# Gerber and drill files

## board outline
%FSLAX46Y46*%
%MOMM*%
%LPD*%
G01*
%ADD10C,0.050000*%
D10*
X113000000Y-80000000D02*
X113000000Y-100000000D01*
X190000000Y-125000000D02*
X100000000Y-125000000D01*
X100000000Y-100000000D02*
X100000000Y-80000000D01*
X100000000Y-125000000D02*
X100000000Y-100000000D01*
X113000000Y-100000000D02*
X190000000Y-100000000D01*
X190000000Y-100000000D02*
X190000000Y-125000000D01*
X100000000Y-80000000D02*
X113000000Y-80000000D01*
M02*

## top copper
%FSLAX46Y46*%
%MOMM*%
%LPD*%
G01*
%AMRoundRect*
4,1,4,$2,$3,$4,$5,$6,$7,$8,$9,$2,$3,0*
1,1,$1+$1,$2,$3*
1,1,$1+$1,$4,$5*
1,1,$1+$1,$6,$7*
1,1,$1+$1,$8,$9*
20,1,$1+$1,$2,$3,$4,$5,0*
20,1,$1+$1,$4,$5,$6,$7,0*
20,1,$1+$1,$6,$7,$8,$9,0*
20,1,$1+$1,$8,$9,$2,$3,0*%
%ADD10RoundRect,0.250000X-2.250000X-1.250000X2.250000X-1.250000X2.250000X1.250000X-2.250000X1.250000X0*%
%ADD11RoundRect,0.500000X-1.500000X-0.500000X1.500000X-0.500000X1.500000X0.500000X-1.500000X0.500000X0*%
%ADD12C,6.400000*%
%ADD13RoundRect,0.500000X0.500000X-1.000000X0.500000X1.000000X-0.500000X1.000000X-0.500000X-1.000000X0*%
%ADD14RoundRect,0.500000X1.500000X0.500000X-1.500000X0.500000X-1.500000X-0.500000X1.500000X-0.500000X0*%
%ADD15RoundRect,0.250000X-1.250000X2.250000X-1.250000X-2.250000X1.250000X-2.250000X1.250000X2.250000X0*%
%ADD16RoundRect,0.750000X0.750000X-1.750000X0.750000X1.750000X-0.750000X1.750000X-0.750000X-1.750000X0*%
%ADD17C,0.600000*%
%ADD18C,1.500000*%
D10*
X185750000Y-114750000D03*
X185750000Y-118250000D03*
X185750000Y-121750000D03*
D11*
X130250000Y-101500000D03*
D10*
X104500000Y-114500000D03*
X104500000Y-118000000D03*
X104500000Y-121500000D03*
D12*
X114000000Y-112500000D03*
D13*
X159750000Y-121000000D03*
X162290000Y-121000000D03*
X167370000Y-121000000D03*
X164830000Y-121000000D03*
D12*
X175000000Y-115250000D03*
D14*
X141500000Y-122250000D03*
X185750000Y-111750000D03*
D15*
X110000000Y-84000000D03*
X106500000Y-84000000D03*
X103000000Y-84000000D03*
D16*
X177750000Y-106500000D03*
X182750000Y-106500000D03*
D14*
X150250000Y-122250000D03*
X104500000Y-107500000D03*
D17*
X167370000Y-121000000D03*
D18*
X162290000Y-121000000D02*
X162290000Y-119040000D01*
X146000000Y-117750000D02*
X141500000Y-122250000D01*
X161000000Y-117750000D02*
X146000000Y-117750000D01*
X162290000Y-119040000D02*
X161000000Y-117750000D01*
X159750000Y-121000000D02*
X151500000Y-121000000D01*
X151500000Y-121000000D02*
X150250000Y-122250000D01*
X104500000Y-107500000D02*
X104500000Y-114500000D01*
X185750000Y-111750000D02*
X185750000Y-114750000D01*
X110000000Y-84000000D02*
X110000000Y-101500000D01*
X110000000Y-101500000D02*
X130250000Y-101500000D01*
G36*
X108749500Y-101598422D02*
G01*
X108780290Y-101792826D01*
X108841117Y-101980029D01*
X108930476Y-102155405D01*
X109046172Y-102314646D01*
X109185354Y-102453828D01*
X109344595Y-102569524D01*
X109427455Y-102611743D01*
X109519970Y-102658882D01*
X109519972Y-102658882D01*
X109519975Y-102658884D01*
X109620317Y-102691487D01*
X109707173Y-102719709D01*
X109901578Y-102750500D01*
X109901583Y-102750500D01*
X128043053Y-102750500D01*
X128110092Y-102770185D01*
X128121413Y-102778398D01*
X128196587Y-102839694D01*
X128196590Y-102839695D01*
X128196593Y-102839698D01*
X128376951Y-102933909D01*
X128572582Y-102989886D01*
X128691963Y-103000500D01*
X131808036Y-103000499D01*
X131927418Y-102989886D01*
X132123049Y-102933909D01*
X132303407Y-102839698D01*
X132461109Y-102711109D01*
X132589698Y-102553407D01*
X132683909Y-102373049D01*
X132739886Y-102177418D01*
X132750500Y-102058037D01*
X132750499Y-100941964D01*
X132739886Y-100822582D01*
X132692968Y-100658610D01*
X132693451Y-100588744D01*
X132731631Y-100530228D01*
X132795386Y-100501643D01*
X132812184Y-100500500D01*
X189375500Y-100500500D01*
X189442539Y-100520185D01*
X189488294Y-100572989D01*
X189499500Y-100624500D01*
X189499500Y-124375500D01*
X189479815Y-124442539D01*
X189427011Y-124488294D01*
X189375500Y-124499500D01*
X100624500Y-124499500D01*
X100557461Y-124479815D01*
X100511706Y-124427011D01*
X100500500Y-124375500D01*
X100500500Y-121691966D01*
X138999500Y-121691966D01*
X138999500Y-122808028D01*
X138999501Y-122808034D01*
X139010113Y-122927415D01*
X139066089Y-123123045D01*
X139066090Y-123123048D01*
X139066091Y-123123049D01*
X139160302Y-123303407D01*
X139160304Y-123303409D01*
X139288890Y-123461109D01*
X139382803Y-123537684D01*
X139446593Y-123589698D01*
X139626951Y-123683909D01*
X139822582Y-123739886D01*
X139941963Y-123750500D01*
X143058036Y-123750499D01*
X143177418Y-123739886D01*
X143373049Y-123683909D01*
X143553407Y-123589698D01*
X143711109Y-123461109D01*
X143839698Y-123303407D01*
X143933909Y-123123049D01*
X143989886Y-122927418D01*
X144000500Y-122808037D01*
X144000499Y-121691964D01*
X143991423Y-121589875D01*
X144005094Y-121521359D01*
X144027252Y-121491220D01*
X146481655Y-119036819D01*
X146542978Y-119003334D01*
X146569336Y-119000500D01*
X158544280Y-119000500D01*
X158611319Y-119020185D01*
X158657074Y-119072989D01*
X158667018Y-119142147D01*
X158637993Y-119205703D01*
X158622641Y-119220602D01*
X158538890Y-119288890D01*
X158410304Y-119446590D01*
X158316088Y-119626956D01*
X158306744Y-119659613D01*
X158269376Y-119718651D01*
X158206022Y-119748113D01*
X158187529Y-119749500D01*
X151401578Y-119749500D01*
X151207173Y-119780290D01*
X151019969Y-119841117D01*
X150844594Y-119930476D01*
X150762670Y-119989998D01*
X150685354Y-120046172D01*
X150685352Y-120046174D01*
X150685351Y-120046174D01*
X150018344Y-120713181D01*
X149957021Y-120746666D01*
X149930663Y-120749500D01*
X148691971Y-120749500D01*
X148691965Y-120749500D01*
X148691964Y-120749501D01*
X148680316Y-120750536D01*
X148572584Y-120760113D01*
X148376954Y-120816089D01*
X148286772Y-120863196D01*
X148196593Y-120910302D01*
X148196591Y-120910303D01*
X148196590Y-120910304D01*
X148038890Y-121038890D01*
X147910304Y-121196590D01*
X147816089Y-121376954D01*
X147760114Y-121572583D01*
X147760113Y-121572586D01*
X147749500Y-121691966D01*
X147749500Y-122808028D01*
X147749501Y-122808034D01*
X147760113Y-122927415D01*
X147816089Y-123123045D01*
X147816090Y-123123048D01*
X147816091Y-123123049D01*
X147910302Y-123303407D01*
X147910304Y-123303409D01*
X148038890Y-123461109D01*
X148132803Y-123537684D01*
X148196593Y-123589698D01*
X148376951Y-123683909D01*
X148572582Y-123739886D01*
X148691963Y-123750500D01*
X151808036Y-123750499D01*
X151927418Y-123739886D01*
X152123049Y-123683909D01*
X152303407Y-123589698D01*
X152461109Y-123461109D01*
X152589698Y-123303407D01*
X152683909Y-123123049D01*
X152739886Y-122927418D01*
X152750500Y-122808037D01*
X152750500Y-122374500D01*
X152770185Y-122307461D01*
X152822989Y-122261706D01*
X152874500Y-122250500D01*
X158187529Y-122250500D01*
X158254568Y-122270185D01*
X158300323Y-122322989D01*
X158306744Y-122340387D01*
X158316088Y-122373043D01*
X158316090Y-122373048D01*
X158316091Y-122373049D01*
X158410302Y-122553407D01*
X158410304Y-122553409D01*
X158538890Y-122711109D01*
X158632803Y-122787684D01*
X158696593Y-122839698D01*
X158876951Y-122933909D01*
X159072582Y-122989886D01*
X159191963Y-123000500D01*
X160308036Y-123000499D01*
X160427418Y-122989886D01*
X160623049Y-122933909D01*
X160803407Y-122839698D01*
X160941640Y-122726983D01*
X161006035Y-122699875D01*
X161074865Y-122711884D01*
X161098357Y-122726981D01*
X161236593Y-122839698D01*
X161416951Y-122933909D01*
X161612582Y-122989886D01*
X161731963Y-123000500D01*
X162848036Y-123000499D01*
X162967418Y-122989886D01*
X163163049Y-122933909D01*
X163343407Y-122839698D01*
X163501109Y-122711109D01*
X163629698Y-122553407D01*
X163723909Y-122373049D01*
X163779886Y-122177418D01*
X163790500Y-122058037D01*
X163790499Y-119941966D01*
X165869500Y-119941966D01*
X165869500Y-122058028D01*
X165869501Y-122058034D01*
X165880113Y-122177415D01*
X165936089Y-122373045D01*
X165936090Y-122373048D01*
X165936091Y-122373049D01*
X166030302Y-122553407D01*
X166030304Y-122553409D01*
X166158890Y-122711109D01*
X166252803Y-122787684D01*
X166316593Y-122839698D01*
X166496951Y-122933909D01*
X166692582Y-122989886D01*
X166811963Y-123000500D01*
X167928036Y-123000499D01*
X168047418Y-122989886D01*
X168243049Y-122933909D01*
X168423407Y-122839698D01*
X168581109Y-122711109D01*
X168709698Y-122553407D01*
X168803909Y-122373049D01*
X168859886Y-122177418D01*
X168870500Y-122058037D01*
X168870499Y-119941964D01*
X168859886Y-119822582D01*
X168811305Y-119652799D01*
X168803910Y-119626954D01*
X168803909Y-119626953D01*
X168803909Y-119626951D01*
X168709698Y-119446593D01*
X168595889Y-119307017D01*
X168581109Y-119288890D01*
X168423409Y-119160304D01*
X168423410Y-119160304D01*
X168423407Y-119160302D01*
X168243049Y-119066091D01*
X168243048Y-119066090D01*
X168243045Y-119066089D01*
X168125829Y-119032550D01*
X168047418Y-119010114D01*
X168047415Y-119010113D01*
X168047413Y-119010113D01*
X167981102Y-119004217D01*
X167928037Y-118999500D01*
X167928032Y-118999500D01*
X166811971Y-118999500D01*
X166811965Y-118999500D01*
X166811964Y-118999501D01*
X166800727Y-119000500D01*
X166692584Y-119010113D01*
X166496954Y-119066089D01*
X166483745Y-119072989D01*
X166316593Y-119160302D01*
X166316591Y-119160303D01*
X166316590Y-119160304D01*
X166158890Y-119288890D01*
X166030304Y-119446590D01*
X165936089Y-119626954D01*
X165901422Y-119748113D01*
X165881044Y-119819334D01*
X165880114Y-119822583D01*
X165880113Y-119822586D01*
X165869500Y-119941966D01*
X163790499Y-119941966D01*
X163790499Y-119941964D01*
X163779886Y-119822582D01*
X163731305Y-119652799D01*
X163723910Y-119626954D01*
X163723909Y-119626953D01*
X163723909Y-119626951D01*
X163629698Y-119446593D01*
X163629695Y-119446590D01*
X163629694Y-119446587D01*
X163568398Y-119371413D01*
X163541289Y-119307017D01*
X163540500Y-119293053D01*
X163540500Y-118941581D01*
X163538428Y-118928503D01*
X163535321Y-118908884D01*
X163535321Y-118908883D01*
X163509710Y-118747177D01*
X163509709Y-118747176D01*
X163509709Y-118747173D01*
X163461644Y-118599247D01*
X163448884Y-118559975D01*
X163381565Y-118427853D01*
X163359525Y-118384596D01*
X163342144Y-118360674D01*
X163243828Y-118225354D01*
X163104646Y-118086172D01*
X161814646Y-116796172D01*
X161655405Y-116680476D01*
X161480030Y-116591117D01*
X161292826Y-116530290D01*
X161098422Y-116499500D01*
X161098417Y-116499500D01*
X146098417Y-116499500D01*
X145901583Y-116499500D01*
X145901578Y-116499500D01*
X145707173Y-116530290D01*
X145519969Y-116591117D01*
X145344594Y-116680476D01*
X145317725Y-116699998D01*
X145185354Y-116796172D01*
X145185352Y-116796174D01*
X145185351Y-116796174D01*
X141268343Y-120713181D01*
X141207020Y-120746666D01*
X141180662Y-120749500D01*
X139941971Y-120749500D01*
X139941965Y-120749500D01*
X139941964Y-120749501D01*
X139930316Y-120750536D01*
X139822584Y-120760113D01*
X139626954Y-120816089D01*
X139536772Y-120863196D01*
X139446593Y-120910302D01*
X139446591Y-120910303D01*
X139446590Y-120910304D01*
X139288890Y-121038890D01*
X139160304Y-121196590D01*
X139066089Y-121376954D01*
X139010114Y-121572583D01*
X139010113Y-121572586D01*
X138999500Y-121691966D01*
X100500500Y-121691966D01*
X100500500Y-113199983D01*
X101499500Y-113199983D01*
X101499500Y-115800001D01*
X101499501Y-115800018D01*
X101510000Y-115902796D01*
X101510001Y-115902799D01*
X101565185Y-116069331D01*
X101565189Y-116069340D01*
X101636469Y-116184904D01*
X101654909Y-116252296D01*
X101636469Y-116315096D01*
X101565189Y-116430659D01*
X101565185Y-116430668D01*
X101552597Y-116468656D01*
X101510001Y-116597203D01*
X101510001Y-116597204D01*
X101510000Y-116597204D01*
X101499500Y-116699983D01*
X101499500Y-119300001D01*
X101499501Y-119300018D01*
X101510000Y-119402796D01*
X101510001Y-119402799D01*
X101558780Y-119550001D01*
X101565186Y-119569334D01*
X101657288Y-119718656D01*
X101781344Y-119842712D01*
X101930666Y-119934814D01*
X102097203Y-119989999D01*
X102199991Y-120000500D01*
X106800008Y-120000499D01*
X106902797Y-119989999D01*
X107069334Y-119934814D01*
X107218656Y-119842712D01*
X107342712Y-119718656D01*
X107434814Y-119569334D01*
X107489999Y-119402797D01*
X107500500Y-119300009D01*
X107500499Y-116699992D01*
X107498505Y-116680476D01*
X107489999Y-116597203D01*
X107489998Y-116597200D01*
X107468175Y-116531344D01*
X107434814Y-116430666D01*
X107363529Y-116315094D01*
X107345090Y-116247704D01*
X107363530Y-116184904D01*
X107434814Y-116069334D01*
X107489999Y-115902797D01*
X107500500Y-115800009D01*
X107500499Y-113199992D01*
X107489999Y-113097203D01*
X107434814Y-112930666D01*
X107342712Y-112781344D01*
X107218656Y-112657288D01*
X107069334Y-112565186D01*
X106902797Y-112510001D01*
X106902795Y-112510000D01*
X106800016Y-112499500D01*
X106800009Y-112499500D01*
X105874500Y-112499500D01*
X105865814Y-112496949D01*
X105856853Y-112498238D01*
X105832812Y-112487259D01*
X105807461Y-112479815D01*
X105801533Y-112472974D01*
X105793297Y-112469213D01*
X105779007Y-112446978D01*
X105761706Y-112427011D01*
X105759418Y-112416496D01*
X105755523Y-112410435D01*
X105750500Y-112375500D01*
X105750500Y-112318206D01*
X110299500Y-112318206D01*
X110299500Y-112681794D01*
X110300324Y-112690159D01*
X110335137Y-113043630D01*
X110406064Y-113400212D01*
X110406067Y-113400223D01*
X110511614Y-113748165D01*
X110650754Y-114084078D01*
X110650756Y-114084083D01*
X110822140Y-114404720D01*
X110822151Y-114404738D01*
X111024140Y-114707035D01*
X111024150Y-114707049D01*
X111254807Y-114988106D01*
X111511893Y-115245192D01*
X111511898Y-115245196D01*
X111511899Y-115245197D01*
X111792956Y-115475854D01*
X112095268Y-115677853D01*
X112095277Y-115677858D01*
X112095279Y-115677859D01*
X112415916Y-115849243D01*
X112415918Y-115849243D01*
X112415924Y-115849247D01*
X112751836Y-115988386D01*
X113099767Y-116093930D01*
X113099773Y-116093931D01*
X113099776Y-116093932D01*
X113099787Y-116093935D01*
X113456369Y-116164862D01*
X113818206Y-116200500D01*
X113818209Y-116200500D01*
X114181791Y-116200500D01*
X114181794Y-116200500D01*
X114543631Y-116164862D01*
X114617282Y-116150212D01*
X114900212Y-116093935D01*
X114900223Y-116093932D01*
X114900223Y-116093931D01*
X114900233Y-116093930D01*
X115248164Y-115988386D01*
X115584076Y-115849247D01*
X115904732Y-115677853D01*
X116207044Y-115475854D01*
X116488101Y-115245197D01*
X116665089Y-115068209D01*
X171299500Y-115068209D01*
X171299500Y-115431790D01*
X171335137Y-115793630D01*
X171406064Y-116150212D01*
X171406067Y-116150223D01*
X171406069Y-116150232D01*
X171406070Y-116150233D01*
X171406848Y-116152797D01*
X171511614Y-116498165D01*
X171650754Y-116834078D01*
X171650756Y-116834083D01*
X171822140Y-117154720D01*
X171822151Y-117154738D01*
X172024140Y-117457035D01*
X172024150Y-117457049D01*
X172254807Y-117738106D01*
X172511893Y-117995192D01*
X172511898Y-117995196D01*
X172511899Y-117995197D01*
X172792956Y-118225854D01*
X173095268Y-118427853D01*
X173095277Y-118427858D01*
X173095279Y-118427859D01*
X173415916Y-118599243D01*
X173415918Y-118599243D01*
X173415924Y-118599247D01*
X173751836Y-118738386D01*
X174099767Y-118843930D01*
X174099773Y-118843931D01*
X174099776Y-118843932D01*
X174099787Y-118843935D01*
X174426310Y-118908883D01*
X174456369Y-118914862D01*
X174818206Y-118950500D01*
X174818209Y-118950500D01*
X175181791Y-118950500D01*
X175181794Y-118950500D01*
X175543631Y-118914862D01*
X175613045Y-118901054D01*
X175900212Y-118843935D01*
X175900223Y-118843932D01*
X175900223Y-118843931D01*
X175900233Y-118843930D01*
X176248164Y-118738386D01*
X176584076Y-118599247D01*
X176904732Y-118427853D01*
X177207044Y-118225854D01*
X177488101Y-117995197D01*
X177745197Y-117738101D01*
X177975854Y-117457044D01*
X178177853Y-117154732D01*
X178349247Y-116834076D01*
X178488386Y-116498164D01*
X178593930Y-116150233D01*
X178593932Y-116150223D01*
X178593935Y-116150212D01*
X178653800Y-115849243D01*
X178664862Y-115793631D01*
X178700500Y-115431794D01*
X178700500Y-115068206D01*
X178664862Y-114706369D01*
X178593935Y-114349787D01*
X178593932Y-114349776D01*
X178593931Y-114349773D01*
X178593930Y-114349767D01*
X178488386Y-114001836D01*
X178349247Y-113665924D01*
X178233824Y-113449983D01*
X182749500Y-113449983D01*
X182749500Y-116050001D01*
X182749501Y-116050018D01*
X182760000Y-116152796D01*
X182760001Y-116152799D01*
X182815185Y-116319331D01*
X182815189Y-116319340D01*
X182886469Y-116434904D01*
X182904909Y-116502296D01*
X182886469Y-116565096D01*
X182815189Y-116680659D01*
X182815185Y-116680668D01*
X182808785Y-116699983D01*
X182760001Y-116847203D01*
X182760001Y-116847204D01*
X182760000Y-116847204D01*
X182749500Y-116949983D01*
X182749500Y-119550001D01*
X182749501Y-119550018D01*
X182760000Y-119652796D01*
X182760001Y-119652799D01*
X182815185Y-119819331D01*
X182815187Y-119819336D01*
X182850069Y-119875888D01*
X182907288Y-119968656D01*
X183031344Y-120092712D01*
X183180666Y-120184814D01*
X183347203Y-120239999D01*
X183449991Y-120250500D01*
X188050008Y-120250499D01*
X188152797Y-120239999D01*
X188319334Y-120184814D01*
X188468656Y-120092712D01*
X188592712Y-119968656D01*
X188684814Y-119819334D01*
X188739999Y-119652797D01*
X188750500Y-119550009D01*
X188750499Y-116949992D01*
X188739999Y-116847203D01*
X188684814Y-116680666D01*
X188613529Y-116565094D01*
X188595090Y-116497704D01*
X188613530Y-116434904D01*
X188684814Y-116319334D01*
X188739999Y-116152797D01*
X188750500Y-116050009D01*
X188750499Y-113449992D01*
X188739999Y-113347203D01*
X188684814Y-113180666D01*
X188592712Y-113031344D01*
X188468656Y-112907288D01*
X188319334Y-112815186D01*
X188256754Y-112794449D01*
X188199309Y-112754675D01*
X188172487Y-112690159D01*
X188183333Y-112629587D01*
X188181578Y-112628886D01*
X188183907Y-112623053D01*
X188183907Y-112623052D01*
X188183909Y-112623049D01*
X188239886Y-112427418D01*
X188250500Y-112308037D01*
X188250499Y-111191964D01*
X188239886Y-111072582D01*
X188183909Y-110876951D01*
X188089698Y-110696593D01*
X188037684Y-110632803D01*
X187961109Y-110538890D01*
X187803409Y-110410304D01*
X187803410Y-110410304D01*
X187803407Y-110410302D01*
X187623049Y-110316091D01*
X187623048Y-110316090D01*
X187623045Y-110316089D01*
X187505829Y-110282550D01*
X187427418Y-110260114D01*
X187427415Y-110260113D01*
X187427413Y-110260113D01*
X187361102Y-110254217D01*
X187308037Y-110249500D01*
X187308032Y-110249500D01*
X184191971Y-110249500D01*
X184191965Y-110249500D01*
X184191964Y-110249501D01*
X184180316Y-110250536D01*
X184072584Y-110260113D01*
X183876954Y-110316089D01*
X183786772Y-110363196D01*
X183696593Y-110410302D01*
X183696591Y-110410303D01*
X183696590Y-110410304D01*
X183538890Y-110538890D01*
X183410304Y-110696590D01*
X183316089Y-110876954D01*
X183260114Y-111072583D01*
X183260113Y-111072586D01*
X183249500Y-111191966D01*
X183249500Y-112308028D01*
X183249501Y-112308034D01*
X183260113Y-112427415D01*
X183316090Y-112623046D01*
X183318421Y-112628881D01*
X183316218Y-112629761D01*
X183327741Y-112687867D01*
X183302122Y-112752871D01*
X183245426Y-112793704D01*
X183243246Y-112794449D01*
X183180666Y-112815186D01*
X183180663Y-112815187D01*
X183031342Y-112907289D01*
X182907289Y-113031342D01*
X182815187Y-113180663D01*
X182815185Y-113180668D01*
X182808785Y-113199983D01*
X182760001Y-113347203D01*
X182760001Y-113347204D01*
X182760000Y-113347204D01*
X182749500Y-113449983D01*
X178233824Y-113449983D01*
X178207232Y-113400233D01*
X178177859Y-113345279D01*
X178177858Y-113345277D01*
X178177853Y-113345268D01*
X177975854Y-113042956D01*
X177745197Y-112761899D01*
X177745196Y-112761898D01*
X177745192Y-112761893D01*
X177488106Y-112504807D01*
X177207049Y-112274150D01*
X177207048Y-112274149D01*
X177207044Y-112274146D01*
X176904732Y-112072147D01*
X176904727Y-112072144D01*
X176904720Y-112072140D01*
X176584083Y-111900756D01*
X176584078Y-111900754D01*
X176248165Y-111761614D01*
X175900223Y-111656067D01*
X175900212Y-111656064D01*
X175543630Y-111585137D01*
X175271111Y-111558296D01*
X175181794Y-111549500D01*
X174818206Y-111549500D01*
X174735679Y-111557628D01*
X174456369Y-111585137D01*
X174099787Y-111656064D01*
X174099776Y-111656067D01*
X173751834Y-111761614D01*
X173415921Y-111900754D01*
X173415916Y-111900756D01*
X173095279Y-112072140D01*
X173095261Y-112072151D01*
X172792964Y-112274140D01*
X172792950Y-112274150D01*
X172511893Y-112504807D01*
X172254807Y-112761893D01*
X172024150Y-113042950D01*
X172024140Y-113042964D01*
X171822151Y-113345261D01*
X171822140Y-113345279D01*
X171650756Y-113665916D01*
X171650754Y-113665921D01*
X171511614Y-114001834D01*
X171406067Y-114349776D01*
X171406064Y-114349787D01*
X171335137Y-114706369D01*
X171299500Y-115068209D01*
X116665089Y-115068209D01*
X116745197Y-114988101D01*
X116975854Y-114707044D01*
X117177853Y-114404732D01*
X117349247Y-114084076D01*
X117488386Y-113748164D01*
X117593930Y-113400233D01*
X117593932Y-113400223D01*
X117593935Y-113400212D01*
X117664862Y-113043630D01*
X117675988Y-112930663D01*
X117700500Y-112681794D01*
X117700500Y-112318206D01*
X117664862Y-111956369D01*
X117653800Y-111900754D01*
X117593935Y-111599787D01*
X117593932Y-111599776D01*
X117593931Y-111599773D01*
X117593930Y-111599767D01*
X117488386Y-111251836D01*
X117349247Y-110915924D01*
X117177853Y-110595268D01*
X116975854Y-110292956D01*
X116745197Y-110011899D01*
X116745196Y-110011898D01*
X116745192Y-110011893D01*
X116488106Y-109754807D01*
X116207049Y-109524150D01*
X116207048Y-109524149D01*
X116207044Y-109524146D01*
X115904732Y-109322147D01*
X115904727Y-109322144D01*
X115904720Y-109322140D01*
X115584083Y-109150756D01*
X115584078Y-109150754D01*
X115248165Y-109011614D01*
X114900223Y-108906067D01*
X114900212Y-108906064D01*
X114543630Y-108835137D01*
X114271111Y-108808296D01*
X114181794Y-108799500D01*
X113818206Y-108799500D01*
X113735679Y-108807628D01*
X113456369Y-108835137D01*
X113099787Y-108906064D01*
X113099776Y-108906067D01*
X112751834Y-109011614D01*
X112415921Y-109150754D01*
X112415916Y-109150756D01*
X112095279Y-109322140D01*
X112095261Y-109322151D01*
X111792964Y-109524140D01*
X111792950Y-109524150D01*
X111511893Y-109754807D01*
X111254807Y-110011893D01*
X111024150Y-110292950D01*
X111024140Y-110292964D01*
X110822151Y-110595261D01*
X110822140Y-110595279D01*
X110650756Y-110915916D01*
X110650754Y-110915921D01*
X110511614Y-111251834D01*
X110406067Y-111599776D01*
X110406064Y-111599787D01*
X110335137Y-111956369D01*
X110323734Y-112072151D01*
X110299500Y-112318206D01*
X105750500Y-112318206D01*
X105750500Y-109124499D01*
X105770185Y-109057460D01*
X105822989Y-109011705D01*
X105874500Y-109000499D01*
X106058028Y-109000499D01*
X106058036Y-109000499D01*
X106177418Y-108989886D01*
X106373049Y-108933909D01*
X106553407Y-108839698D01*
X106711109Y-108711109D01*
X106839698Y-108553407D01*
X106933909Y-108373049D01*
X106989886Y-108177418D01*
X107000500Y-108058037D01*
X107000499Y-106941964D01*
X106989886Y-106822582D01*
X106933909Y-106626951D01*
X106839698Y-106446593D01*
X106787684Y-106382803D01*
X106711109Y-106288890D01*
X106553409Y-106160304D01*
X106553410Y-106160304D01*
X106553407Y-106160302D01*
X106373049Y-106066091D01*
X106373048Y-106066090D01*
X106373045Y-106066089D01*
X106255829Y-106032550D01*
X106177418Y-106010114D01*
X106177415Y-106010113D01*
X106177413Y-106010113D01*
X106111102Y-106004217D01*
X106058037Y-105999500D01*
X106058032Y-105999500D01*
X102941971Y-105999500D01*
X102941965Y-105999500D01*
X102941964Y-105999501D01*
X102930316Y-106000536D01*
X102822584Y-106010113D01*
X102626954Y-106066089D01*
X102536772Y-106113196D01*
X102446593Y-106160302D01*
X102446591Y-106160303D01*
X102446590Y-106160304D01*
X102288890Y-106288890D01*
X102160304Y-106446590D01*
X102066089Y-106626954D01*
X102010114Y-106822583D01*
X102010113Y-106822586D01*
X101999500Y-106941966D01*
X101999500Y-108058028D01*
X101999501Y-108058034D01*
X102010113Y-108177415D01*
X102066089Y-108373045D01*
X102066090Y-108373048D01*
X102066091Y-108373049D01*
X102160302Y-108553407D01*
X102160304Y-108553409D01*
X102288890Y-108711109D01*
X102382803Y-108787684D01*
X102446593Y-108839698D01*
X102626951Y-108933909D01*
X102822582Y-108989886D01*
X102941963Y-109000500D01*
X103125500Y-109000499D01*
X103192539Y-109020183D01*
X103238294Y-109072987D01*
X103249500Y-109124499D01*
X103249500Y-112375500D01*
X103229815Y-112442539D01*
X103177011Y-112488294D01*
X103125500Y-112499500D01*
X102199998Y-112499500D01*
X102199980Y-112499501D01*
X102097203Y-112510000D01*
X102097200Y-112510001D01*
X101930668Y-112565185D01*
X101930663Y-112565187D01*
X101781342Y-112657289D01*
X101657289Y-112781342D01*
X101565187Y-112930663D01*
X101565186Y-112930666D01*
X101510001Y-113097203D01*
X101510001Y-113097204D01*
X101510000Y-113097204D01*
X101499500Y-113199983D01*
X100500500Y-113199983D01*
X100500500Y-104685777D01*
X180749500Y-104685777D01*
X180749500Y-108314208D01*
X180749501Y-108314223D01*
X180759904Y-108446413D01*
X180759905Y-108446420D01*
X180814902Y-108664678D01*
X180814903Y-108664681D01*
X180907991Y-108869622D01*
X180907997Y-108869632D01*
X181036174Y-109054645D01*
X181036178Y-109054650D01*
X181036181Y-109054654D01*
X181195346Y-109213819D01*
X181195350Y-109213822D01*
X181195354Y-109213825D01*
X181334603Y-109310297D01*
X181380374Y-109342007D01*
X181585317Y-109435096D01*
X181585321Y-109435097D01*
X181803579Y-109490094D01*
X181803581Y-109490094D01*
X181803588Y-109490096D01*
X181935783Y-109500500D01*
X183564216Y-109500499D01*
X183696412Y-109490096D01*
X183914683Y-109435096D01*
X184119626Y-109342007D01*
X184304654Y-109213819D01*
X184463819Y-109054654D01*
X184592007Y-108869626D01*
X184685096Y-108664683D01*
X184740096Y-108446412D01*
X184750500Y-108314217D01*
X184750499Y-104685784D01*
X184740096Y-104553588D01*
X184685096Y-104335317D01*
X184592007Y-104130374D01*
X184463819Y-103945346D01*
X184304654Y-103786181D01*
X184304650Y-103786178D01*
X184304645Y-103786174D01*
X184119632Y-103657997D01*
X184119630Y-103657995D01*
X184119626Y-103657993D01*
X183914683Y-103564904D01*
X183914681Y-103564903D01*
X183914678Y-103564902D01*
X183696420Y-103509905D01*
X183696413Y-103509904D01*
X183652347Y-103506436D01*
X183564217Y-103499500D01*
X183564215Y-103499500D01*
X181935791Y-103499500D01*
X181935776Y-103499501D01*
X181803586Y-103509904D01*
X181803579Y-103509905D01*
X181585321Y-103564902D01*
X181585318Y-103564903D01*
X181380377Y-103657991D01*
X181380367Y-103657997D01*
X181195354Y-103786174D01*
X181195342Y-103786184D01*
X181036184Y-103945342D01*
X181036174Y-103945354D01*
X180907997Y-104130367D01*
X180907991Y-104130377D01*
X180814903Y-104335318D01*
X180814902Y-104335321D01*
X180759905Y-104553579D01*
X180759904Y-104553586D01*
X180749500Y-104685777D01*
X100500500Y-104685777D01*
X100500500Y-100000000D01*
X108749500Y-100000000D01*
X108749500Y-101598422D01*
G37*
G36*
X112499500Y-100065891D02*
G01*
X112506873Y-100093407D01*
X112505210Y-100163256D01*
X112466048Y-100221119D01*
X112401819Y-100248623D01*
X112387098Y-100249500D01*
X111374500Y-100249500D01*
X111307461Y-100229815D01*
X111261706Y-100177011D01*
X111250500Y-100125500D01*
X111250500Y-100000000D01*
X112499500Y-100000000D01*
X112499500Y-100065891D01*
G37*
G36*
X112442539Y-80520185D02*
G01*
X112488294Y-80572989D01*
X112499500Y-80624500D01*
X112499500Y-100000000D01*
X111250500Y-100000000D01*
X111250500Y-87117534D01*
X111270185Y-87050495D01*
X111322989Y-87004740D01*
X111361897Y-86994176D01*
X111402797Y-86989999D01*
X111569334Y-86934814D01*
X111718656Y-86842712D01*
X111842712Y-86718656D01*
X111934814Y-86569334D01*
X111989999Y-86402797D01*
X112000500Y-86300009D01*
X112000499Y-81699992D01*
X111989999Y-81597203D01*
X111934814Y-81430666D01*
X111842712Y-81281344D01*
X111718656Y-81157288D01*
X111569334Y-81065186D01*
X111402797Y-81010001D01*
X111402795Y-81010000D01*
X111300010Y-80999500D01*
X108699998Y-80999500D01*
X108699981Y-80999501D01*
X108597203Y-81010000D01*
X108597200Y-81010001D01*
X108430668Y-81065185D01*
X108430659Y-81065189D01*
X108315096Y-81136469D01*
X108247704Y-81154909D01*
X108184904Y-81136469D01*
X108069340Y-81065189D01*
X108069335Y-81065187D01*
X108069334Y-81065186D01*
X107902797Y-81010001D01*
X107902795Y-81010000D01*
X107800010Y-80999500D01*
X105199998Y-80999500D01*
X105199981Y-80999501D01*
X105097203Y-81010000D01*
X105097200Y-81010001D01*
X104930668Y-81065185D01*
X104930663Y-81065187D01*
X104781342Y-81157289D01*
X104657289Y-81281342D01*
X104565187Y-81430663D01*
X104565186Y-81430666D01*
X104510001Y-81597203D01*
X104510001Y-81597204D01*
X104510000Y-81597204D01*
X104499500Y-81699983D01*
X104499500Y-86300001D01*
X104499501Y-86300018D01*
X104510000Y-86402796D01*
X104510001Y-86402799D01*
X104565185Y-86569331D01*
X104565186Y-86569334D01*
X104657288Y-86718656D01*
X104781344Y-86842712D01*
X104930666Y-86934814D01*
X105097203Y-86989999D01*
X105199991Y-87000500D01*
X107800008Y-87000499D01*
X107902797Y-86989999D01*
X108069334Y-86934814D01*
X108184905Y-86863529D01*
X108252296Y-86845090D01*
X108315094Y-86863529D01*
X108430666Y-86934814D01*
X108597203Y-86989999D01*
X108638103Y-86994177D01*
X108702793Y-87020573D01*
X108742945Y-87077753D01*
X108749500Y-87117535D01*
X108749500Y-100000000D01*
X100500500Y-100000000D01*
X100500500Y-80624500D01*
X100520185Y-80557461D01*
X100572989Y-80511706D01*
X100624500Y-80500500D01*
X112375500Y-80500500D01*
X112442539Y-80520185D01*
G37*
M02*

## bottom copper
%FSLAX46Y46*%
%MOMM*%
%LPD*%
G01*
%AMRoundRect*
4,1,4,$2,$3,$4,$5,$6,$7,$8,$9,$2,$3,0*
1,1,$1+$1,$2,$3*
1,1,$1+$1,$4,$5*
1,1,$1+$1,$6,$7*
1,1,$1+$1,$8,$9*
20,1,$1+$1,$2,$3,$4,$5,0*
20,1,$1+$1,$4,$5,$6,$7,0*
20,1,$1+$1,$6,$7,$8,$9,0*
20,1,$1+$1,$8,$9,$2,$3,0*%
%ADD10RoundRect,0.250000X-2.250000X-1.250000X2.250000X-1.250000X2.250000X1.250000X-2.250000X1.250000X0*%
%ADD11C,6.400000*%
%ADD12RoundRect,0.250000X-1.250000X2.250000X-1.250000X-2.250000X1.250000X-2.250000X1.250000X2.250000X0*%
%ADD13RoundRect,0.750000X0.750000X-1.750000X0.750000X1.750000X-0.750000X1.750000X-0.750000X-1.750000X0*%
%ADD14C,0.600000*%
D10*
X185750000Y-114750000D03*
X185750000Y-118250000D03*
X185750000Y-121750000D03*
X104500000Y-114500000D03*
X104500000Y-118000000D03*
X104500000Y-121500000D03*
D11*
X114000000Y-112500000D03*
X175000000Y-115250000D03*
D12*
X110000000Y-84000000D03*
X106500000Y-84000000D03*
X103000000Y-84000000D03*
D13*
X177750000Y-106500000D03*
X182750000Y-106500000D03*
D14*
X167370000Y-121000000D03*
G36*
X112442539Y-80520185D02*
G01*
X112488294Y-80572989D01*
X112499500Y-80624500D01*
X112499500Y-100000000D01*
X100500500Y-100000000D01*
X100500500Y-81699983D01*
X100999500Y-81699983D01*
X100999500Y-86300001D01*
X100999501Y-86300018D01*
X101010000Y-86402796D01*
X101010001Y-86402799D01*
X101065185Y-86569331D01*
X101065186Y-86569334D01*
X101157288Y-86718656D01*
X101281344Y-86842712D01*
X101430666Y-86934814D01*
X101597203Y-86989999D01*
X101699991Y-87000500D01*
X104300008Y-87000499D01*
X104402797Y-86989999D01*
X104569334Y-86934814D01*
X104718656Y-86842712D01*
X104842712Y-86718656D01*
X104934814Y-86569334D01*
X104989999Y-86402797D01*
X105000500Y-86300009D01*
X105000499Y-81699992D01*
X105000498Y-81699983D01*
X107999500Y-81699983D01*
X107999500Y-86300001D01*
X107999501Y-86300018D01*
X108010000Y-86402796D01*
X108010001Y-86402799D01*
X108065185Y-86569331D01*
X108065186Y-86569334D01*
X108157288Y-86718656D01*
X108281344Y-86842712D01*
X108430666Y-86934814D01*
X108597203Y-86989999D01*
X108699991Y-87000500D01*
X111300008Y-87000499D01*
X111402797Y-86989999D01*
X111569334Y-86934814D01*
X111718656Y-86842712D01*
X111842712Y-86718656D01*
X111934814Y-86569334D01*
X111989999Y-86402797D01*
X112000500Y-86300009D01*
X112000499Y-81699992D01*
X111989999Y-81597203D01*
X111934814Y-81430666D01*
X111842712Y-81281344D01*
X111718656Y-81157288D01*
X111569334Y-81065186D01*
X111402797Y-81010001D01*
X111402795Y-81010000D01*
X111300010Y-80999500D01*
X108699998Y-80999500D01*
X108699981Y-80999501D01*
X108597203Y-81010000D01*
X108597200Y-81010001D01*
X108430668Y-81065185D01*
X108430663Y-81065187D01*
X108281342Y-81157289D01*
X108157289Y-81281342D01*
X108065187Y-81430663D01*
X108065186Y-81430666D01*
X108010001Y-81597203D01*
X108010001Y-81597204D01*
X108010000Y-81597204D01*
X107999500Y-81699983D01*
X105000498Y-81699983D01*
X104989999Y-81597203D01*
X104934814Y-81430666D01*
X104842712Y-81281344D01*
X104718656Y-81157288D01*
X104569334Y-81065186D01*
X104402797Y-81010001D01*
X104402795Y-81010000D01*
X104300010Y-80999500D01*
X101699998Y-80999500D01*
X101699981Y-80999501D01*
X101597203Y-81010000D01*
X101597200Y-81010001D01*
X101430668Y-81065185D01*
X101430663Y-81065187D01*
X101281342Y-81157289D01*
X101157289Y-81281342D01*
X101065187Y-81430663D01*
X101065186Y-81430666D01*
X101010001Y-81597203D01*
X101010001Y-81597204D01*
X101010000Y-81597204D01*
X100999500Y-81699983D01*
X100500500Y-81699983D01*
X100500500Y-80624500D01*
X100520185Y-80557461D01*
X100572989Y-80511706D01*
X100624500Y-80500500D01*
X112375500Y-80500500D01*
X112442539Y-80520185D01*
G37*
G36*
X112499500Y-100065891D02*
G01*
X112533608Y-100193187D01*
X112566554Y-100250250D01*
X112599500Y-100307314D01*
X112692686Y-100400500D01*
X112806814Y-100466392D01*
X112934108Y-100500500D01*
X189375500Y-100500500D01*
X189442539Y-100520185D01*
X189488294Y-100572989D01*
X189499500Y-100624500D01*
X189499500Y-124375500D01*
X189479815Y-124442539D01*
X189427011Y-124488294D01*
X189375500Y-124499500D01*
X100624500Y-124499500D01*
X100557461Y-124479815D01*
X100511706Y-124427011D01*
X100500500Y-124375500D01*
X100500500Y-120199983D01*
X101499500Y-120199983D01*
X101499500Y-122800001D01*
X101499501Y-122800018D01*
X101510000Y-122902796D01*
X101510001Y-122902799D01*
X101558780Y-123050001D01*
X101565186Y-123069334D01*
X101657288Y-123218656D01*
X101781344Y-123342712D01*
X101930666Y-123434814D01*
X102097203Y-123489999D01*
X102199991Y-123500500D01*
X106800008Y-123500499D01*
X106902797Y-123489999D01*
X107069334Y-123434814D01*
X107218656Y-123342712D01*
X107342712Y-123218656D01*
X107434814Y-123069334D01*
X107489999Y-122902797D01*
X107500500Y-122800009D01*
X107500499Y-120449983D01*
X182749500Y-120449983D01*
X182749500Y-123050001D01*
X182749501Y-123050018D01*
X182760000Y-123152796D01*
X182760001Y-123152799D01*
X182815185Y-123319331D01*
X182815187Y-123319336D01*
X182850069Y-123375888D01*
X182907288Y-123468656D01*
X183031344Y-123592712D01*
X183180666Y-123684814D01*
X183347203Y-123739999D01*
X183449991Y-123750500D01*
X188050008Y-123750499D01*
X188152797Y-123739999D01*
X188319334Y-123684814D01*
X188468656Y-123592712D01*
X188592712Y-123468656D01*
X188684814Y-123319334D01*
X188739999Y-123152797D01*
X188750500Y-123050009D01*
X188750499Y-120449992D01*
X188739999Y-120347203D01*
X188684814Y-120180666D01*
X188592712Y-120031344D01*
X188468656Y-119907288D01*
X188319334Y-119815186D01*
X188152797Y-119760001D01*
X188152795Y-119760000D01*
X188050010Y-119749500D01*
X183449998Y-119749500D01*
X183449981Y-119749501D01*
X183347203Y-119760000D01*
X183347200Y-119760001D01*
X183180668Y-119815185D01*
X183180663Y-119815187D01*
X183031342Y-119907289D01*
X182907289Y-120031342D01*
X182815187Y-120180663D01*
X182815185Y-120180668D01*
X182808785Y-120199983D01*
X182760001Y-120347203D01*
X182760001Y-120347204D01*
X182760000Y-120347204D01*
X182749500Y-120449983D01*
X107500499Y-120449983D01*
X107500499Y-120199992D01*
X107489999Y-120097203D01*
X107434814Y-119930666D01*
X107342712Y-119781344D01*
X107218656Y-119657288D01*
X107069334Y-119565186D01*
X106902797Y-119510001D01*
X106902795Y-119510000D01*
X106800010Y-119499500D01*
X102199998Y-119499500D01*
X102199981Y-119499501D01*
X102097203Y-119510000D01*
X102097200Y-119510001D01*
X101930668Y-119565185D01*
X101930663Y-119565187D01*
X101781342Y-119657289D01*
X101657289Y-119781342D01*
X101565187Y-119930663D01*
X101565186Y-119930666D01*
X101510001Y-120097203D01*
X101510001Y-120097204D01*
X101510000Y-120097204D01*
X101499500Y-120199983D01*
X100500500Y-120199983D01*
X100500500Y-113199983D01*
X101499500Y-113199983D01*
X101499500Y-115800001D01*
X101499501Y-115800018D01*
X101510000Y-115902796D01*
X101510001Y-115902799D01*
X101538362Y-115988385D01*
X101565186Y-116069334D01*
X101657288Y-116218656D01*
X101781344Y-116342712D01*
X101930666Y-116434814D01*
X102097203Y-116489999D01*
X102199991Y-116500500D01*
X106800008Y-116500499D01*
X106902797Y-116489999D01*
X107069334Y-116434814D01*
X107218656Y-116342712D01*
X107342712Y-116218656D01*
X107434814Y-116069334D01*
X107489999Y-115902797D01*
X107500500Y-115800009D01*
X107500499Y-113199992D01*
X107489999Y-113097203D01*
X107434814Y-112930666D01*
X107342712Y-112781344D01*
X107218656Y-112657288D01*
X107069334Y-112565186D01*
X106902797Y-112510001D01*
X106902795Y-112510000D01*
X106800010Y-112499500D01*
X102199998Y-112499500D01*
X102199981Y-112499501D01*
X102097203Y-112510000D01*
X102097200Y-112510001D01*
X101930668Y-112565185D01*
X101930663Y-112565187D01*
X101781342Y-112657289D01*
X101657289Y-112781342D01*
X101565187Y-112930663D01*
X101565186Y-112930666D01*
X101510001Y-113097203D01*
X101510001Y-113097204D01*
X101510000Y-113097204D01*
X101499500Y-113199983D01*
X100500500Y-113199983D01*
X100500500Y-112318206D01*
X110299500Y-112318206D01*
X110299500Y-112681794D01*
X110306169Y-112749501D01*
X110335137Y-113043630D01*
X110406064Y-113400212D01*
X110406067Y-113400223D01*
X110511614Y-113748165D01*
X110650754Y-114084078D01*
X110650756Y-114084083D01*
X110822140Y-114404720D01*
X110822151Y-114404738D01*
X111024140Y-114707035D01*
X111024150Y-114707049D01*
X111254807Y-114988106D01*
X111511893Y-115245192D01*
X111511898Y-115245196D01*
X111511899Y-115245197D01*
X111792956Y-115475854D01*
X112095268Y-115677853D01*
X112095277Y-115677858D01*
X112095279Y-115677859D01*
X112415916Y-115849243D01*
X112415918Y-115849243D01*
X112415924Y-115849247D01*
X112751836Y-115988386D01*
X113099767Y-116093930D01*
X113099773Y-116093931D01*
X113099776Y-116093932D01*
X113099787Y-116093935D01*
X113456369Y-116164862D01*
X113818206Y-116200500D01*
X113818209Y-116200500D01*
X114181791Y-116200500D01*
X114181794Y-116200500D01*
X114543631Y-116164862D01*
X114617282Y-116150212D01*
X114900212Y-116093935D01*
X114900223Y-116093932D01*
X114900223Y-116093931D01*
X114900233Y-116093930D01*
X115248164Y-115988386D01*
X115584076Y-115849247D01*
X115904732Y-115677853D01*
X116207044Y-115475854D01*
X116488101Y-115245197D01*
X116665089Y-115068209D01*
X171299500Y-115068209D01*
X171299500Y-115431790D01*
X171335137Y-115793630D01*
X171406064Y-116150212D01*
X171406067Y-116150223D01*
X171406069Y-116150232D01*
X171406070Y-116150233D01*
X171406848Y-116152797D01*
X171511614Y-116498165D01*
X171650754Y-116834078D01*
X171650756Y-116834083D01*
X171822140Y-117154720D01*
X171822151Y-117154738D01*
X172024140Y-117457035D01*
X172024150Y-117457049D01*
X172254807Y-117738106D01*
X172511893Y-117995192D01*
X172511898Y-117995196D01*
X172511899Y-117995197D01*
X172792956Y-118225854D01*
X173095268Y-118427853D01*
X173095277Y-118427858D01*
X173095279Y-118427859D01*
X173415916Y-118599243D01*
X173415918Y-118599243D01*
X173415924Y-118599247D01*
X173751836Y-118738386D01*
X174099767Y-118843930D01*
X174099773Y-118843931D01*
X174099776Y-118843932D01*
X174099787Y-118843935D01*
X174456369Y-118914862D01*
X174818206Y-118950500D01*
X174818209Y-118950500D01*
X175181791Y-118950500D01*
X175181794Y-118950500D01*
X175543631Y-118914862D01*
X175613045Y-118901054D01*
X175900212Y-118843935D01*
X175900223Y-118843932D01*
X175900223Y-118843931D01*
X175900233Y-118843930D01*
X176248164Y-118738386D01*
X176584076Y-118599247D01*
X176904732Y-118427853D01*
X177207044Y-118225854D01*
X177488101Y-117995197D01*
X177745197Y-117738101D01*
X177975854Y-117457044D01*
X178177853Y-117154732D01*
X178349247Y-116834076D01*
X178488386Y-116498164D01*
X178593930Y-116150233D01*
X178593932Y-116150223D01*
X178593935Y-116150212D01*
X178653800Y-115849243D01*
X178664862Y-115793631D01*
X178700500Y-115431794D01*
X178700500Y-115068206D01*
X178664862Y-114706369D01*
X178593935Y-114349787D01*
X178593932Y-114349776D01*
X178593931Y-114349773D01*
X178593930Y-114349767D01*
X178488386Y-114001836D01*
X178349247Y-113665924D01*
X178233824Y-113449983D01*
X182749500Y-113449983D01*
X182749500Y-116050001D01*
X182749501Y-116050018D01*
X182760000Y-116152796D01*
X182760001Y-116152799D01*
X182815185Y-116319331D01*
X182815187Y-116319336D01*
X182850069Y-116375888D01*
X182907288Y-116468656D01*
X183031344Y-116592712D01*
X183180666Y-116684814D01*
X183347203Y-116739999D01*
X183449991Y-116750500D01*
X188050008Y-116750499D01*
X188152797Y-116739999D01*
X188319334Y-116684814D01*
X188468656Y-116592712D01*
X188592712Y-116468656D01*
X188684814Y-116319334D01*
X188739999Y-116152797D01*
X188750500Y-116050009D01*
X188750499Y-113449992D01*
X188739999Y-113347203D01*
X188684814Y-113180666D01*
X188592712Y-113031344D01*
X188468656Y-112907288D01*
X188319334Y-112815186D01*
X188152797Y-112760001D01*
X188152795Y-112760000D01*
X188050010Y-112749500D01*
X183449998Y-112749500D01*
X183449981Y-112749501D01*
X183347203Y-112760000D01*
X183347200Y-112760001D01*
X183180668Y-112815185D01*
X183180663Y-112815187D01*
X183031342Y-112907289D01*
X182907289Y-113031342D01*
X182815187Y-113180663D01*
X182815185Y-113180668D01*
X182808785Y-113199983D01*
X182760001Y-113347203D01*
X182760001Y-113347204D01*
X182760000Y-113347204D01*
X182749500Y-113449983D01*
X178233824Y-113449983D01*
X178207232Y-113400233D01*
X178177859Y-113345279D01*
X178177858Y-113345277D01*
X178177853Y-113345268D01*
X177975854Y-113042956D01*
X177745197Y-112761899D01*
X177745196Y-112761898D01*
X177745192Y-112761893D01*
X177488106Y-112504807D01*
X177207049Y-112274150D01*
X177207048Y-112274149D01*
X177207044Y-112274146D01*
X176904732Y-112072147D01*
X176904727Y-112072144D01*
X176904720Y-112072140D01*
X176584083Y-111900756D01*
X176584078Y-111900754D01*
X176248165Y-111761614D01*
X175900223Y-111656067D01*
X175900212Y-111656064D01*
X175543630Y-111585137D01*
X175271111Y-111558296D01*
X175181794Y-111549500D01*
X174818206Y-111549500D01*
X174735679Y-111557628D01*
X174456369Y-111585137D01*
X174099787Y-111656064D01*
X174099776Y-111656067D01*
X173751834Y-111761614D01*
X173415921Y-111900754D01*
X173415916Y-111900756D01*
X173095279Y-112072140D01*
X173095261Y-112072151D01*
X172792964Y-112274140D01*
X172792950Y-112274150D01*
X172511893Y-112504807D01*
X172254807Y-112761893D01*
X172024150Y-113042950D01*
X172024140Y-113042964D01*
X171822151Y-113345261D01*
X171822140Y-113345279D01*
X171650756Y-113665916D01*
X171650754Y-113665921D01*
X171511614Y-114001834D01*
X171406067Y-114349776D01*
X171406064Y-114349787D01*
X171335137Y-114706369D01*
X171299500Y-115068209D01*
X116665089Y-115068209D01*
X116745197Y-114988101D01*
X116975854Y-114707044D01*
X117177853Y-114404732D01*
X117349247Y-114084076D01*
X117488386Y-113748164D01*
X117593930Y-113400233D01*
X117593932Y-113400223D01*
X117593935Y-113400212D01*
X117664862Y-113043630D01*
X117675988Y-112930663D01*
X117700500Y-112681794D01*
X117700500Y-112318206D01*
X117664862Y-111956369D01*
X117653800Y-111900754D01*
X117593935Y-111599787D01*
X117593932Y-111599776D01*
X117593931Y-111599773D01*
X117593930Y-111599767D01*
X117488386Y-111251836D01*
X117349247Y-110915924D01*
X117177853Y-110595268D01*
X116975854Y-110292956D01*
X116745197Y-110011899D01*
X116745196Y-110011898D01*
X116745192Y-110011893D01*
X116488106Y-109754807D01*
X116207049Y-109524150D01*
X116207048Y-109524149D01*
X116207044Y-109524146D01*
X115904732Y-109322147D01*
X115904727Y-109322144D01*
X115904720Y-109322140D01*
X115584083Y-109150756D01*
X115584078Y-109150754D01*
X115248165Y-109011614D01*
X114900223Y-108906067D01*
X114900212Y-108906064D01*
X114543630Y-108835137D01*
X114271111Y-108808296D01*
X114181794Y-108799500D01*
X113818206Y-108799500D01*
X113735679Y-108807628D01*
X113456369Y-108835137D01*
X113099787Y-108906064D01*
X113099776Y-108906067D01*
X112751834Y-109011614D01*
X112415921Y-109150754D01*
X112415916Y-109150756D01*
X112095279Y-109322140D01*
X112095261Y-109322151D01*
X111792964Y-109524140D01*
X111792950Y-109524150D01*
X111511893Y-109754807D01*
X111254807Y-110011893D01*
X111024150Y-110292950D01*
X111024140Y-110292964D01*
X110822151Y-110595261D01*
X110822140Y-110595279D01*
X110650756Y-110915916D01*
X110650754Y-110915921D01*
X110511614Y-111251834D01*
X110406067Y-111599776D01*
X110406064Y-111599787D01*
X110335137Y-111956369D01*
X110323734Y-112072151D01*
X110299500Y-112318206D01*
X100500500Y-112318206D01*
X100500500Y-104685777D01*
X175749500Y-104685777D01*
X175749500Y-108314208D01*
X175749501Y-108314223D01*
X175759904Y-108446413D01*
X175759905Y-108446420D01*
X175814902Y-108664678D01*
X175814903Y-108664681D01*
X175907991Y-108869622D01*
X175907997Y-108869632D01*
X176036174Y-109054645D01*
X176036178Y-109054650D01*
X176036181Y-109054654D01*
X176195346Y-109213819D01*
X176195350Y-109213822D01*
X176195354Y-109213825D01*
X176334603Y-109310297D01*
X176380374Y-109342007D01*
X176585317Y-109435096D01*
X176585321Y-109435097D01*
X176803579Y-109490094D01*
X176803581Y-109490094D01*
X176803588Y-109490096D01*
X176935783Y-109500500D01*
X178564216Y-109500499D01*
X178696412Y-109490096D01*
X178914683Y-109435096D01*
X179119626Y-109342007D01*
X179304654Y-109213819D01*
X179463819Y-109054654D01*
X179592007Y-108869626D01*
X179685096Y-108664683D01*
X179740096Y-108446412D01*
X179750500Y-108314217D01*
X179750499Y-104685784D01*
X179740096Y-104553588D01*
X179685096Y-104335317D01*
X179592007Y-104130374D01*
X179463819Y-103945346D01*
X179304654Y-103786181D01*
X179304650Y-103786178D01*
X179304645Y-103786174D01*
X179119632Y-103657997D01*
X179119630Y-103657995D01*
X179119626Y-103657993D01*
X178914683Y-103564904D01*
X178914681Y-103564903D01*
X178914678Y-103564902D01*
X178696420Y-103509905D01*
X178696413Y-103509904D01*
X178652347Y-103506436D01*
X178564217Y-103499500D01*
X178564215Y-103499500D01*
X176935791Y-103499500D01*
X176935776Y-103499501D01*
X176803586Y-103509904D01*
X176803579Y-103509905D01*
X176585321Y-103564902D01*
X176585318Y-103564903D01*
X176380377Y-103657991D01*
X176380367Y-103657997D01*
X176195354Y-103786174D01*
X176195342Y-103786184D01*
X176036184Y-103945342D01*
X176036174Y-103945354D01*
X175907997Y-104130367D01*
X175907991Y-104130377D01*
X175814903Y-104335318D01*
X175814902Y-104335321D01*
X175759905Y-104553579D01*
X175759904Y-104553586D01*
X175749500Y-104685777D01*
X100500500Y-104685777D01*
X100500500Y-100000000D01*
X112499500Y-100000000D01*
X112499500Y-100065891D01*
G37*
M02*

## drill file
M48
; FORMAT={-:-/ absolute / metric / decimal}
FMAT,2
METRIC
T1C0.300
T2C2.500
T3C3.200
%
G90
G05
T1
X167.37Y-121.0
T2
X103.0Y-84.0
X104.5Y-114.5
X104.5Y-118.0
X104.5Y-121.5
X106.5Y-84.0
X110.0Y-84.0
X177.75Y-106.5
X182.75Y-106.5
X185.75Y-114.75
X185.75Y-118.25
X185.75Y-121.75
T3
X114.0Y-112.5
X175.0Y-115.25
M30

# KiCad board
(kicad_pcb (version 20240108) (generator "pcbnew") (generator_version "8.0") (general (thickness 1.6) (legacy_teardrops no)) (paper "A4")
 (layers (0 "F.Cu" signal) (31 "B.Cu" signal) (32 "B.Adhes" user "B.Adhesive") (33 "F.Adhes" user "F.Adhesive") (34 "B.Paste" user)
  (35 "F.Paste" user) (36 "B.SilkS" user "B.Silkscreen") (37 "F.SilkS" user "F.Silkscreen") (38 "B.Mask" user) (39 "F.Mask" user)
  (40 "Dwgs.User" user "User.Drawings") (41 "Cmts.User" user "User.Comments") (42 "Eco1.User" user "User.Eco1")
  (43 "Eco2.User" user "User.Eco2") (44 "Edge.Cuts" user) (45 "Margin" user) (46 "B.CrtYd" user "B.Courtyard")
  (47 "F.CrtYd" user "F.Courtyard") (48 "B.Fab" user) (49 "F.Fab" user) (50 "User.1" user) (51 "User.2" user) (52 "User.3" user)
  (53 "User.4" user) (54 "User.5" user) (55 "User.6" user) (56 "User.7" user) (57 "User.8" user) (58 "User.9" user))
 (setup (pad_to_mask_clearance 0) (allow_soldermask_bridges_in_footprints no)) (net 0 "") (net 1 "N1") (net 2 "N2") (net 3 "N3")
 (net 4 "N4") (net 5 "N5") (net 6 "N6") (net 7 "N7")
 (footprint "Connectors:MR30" (layer "F.Cu") (at 185.75 114.75)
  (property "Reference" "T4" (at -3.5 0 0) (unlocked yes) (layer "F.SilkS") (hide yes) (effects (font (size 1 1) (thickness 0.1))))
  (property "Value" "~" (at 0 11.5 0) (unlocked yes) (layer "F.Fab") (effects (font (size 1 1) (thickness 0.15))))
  (pad "1" thru_hole roundrect (at 0 0) (size 5 3) (drill 2.5) (layers "*.Cu" "*.Mask") (remove_unused_layers no)
   (roundrect_rratio 0.08333333333) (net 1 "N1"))
  (pad "2" thru_hole roundrect (at 0 3.5) (size 5 3) (drill 2.5) (layers "*.Cu" "*.Mask") (remove_unused_layers no)
   (roundrect_rratio 0.08333333333) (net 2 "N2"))
  (pad "3" thru_hole roundrect (at 0 7) (size 5 3) (drill 2.5) (layers "*.Cu" "*.Mask") (remove_unused_layers no)
   (roundrect_rratio 0.08333333333) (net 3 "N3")))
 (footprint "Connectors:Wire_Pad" (layer "F.Cu") (at 130.25 101.5)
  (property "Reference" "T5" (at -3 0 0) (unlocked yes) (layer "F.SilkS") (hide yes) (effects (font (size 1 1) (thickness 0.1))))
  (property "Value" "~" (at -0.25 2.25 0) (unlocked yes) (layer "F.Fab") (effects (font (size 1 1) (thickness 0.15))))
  (pad "1" smd roundrect (at 0 0) (size 4 2) (layers "F.Cu" "F.Paste" "F.Mask") (roundrect_rratio 0.25) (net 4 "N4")
   (thermal_bridge_angle 45)))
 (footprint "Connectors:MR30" (layer "F.Cu") (at 104.5 114.5)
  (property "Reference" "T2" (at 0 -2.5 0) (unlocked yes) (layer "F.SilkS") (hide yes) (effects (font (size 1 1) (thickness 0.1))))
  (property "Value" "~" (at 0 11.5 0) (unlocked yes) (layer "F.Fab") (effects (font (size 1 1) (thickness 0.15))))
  (pad "1" thru_hole roundrect (at 0 0) (size 5 3) (drill 2.5) (layers "*.Cu" "*.Mask") (remove_unused_layers no)
   (roundrect_rratio 0.08333333333) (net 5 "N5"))
  (pad "2" thru_hole roundrect (at 0 3.5) (size 5 3) (drill 2.5) (layers "*.Cu" "*.Mask") (remove_unused_layers no)
   (roundrect_rratio 0.08333333333) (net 2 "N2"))
  (pad "3" thru_hole roundrect (at 0 7) (size 5 3) (drill 2.5) (layers "*.Cu" "*.Mask") (remove_unused_layers no)
   (roundrect_rratio 0.08333333333) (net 3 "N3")))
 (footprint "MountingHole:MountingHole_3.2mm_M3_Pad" (layer "F.Cu") (at 114 112.5)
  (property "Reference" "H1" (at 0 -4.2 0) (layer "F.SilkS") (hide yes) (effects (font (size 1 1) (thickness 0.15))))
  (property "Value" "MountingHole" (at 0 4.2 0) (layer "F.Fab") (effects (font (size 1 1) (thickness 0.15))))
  (pad "1" thru_hole circle (at 0 0) (size 6.4 6.4) (drill 3.2) (layers "*.Cu" "*.Mask") (remove_unused_layers no)))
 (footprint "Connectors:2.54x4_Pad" (layer "F.Cu") (at 159.75 121 90)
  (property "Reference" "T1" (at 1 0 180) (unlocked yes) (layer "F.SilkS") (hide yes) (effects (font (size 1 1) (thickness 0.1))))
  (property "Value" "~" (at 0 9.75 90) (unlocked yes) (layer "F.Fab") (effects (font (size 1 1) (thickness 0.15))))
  (pad "1" smd roundrect (at 0 0 90) (size 3 2) (layers "F.Cu" "F.Paste" "F.Mask") (roundrect_rratio 0.25) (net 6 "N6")
   (thermal_bridge_angle 45))
  (pad "2" smd roundrect (at 0 2.54 90) (size 3 2) (layers "F.Cu" "F.Paste" "F.Mask") (roundrect_rratio 0.25) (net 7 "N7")
   (thermal_bridge_angle 45))
  (pad "3" smd roundrect (at 0 7.62 90) (size 3 2) (layers "F.Cu" "F.Paste" "F.Mask") (roundrect_rratio 0.25) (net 2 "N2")
   (thermal_bridge_angle 45))
  (pad "4" smd roundrect (at 0 5.08 90) (size 3 2) (layers "F.Cu" "F.Paste" "F.Mask") (roundrect_rratio 0.25) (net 3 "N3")
   (thermal_bridge_angle 45)))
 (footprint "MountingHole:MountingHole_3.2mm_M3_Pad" (layer "F.Cu") (at 175 115.25)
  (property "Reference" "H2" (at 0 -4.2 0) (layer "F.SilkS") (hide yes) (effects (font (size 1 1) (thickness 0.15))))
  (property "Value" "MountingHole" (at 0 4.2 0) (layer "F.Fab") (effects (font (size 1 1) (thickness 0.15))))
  (pad "1" thru_hole circle (at 0 0) (size 6.4 6.4) (drill 3.2) (layers "*.Cu" "*.Mask") (remove_unused_layers no)))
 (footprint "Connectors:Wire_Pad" (layer "F.Cu") (at 141.5 122.25 180)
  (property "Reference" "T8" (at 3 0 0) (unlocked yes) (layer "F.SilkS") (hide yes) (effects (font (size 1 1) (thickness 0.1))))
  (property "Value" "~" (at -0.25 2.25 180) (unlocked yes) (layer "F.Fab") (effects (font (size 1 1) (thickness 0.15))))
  (pad "1" smd roundrect (at 0 0 180) (size 4 2) (layers "F.Cu" "F.Paste" "F.Mask") (roundrect_rratio 0.25) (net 7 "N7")
   (thermal_bridge_angle 45)))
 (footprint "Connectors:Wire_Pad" (layer "F.Cu") (at 185.75 111.75 180)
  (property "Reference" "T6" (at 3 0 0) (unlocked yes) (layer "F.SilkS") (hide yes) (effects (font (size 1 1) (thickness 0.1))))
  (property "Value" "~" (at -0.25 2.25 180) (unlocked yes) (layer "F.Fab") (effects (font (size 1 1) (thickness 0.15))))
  (pad "1" smd roundrect (at 0 0 180) (size 4 2) (layers "F.Cu" "F.Paste" "F.Mask") (roundrect_rratio 0.25) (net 1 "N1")
   (thermal_bridge_angle 45)))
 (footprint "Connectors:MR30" (layer "F.Cu") (at 110 84 -90)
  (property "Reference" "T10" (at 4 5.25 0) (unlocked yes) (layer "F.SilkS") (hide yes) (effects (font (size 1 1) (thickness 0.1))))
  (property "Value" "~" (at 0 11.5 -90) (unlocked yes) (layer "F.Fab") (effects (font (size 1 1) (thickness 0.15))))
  (pad "1" thru_hole roundrect (at 0 0 270) (size 5 3) (drill 2.5) (layers "*.Cu" "*.Mask") (remove_unused_layers no)
   (roundrect_rratio 0.08333333333) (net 4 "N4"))
  (pad "2" thru_hole roundrect (at 0 3.5 270) (size 5 3) (drill 2.5) (layers "*.Cu" "*.Mask") (remove_unused_layers no)
   (roundrect_rratio 0.08333333333) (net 2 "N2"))
  (pad "3" thru_hole roundrect (at 0 7 270) (size 5 3) (drill 2.5) (layers "*.Cu" "*.Mask") (remove_unused_layers no)
   (roundrect_rratio 0.08333333333) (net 3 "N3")))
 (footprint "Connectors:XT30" (layer "F.Cu") (at 177.75 106.5 90)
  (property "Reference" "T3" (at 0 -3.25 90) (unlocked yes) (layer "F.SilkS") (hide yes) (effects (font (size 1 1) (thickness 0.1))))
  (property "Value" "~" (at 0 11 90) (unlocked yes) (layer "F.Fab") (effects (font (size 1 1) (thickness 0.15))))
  (pad "1" thru_hole roundrect (at 0 0 90) (size 5 3) (drill 2.5) (layers "*.Cu" "*.Mask") (remove_unused_layers no) (roundrect_rratio 0.25)
   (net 3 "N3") (thermal_bridge_angle 45))
  (pad "2" thru_hole roundrect (at 0 5 90) (size 5 3) (drill 2.5) (layers "*.Cu" "*.Mask") (remove_unused_layers no) (roundrect_rratio 0.25)
   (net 2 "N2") (thermal_bridge_angle 45)))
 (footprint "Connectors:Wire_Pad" (layer "F.Cu") (at 150.25 122.25 180)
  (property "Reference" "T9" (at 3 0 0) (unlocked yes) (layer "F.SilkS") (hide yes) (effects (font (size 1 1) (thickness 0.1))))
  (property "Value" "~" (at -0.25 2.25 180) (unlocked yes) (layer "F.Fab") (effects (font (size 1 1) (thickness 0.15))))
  (pad "1" smd roundrect (at 0 0 180) (size 4 2) (layers "F.Cu" "F.Paste" "F.Mask") (roundrect_rratio 0.25) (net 6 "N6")
   (thermal_bridge_angle 45)))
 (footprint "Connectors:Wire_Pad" (layer "F.Cu") (at 104.5 107.5 180)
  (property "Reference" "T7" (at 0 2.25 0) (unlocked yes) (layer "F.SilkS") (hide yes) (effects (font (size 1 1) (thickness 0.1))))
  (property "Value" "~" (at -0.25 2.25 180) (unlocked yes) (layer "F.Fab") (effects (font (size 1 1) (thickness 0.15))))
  (pad "1" smd roundrect (at 0 0 180) (size 4 2) (layers "F.Cu" "F.Paste" "F.Mask") (roundrect_rratio 0.25) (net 5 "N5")
   (thermal_bridge_angle 45)))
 (gr_line (start 113 80) (end 113 100) (stroke (width 0.05) (type default)) (layer "Edge.Cuts"))
 (gr_line (start 190 125) (end 100 125) (stroke (width 0.05) (type default)) (layer "Edge.Cuts"))
 (gr_line (start 100 100) (end 100 80) (stroke (width 0.05) (type default)) (layer "Edge.Cuts"))
 (gr_line (start 100 125) (end 100 100) (stroke (width 0.05) (type default)) (layer "Edge.Cuts"))
 (gr_line (start 113 100) (end 190 100) (stroke (width 0.05) (type default)) (layer "Edge.Cuts"))
 (gr_line (start 190 100) (end 190 125) (stroke (width 0.05) (type default)) (layer "Edge.Cuts"))
 (gr_line (start 100 80) (end 113 80) (stroke (width 0.05) (type default)) (layer "Edge.Cuts"))
 (segment (start 162.29 121) (end 162.29 119.04) (width 1.5) (layer "F.Cu") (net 7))
 (segment (start 146 117.75) (end 141.5 122.25) (width 1.5) (layer "F.Cu") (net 7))
 (segment (start 161 117.75) (end 146 117.75) (width 1.5) (layer "F.Cu") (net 7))
 (segment (start 162.29 119.04) (end 161 117.75) (width 1.5) (layer "F.Cu") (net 7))
 (via (at 167.37 121) (size 0.6) (drill 0.3) (layers "F.Cu" "B.Cu") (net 2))
 (segment (start 159.75 121) (end 151.5 121) (width 1.5) (layer "F.Cu") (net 6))
 (segment (start 151.5 121) (end 150.25 122.25) (width 1.5) (layer "F.Cu") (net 6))
 (segment (start 104.5 107.5) (end 104.5 114.5) (width 1.5) (layer "F.Cu") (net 5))
 (segment (start 185.75 111.75) (end 185.75 114.75) (width 1.5) (layer "F.Cu") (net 1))
 (segment (start 110 84) (end 110 101.5) (width 1.5) (layer "F.Cu") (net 4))
 (segment (start 110 101.5) (end 130.25 101.5) (width 1.5) (layer "F.Cu") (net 4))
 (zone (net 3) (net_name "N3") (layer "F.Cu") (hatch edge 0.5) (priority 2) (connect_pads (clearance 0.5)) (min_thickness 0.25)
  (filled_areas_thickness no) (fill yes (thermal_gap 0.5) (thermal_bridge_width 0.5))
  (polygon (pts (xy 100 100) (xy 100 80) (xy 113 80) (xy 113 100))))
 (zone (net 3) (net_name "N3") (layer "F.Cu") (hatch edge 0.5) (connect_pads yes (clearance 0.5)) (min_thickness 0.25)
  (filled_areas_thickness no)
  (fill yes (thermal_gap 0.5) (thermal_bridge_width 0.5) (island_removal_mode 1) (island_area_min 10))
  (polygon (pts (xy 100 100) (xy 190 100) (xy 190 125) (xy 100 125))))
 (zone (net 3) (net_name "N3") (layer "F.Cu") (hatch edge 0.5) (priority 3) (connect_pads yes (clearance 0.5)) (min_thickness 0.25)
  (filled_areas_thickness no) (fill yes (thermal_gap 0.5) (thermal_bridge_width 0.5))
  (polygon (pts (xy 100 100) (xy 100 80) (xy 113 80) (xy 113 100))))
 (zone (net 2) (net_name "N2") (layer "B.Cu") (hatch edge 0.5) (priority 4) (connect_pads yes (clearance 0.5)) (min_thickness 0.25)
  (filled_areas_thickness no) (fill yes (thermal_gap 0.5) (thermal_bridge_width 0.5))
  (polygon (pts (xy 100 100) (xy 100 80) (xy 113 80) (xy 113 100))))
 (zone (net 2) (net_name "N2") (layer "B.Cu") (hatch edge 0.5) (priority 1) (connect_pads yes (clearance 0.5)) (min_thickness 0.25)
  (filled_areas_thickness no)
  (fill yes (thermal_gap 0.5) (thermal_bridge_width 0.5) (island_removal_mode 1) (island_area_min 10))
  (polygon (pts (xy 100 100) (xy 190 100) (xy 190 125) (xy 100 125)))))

